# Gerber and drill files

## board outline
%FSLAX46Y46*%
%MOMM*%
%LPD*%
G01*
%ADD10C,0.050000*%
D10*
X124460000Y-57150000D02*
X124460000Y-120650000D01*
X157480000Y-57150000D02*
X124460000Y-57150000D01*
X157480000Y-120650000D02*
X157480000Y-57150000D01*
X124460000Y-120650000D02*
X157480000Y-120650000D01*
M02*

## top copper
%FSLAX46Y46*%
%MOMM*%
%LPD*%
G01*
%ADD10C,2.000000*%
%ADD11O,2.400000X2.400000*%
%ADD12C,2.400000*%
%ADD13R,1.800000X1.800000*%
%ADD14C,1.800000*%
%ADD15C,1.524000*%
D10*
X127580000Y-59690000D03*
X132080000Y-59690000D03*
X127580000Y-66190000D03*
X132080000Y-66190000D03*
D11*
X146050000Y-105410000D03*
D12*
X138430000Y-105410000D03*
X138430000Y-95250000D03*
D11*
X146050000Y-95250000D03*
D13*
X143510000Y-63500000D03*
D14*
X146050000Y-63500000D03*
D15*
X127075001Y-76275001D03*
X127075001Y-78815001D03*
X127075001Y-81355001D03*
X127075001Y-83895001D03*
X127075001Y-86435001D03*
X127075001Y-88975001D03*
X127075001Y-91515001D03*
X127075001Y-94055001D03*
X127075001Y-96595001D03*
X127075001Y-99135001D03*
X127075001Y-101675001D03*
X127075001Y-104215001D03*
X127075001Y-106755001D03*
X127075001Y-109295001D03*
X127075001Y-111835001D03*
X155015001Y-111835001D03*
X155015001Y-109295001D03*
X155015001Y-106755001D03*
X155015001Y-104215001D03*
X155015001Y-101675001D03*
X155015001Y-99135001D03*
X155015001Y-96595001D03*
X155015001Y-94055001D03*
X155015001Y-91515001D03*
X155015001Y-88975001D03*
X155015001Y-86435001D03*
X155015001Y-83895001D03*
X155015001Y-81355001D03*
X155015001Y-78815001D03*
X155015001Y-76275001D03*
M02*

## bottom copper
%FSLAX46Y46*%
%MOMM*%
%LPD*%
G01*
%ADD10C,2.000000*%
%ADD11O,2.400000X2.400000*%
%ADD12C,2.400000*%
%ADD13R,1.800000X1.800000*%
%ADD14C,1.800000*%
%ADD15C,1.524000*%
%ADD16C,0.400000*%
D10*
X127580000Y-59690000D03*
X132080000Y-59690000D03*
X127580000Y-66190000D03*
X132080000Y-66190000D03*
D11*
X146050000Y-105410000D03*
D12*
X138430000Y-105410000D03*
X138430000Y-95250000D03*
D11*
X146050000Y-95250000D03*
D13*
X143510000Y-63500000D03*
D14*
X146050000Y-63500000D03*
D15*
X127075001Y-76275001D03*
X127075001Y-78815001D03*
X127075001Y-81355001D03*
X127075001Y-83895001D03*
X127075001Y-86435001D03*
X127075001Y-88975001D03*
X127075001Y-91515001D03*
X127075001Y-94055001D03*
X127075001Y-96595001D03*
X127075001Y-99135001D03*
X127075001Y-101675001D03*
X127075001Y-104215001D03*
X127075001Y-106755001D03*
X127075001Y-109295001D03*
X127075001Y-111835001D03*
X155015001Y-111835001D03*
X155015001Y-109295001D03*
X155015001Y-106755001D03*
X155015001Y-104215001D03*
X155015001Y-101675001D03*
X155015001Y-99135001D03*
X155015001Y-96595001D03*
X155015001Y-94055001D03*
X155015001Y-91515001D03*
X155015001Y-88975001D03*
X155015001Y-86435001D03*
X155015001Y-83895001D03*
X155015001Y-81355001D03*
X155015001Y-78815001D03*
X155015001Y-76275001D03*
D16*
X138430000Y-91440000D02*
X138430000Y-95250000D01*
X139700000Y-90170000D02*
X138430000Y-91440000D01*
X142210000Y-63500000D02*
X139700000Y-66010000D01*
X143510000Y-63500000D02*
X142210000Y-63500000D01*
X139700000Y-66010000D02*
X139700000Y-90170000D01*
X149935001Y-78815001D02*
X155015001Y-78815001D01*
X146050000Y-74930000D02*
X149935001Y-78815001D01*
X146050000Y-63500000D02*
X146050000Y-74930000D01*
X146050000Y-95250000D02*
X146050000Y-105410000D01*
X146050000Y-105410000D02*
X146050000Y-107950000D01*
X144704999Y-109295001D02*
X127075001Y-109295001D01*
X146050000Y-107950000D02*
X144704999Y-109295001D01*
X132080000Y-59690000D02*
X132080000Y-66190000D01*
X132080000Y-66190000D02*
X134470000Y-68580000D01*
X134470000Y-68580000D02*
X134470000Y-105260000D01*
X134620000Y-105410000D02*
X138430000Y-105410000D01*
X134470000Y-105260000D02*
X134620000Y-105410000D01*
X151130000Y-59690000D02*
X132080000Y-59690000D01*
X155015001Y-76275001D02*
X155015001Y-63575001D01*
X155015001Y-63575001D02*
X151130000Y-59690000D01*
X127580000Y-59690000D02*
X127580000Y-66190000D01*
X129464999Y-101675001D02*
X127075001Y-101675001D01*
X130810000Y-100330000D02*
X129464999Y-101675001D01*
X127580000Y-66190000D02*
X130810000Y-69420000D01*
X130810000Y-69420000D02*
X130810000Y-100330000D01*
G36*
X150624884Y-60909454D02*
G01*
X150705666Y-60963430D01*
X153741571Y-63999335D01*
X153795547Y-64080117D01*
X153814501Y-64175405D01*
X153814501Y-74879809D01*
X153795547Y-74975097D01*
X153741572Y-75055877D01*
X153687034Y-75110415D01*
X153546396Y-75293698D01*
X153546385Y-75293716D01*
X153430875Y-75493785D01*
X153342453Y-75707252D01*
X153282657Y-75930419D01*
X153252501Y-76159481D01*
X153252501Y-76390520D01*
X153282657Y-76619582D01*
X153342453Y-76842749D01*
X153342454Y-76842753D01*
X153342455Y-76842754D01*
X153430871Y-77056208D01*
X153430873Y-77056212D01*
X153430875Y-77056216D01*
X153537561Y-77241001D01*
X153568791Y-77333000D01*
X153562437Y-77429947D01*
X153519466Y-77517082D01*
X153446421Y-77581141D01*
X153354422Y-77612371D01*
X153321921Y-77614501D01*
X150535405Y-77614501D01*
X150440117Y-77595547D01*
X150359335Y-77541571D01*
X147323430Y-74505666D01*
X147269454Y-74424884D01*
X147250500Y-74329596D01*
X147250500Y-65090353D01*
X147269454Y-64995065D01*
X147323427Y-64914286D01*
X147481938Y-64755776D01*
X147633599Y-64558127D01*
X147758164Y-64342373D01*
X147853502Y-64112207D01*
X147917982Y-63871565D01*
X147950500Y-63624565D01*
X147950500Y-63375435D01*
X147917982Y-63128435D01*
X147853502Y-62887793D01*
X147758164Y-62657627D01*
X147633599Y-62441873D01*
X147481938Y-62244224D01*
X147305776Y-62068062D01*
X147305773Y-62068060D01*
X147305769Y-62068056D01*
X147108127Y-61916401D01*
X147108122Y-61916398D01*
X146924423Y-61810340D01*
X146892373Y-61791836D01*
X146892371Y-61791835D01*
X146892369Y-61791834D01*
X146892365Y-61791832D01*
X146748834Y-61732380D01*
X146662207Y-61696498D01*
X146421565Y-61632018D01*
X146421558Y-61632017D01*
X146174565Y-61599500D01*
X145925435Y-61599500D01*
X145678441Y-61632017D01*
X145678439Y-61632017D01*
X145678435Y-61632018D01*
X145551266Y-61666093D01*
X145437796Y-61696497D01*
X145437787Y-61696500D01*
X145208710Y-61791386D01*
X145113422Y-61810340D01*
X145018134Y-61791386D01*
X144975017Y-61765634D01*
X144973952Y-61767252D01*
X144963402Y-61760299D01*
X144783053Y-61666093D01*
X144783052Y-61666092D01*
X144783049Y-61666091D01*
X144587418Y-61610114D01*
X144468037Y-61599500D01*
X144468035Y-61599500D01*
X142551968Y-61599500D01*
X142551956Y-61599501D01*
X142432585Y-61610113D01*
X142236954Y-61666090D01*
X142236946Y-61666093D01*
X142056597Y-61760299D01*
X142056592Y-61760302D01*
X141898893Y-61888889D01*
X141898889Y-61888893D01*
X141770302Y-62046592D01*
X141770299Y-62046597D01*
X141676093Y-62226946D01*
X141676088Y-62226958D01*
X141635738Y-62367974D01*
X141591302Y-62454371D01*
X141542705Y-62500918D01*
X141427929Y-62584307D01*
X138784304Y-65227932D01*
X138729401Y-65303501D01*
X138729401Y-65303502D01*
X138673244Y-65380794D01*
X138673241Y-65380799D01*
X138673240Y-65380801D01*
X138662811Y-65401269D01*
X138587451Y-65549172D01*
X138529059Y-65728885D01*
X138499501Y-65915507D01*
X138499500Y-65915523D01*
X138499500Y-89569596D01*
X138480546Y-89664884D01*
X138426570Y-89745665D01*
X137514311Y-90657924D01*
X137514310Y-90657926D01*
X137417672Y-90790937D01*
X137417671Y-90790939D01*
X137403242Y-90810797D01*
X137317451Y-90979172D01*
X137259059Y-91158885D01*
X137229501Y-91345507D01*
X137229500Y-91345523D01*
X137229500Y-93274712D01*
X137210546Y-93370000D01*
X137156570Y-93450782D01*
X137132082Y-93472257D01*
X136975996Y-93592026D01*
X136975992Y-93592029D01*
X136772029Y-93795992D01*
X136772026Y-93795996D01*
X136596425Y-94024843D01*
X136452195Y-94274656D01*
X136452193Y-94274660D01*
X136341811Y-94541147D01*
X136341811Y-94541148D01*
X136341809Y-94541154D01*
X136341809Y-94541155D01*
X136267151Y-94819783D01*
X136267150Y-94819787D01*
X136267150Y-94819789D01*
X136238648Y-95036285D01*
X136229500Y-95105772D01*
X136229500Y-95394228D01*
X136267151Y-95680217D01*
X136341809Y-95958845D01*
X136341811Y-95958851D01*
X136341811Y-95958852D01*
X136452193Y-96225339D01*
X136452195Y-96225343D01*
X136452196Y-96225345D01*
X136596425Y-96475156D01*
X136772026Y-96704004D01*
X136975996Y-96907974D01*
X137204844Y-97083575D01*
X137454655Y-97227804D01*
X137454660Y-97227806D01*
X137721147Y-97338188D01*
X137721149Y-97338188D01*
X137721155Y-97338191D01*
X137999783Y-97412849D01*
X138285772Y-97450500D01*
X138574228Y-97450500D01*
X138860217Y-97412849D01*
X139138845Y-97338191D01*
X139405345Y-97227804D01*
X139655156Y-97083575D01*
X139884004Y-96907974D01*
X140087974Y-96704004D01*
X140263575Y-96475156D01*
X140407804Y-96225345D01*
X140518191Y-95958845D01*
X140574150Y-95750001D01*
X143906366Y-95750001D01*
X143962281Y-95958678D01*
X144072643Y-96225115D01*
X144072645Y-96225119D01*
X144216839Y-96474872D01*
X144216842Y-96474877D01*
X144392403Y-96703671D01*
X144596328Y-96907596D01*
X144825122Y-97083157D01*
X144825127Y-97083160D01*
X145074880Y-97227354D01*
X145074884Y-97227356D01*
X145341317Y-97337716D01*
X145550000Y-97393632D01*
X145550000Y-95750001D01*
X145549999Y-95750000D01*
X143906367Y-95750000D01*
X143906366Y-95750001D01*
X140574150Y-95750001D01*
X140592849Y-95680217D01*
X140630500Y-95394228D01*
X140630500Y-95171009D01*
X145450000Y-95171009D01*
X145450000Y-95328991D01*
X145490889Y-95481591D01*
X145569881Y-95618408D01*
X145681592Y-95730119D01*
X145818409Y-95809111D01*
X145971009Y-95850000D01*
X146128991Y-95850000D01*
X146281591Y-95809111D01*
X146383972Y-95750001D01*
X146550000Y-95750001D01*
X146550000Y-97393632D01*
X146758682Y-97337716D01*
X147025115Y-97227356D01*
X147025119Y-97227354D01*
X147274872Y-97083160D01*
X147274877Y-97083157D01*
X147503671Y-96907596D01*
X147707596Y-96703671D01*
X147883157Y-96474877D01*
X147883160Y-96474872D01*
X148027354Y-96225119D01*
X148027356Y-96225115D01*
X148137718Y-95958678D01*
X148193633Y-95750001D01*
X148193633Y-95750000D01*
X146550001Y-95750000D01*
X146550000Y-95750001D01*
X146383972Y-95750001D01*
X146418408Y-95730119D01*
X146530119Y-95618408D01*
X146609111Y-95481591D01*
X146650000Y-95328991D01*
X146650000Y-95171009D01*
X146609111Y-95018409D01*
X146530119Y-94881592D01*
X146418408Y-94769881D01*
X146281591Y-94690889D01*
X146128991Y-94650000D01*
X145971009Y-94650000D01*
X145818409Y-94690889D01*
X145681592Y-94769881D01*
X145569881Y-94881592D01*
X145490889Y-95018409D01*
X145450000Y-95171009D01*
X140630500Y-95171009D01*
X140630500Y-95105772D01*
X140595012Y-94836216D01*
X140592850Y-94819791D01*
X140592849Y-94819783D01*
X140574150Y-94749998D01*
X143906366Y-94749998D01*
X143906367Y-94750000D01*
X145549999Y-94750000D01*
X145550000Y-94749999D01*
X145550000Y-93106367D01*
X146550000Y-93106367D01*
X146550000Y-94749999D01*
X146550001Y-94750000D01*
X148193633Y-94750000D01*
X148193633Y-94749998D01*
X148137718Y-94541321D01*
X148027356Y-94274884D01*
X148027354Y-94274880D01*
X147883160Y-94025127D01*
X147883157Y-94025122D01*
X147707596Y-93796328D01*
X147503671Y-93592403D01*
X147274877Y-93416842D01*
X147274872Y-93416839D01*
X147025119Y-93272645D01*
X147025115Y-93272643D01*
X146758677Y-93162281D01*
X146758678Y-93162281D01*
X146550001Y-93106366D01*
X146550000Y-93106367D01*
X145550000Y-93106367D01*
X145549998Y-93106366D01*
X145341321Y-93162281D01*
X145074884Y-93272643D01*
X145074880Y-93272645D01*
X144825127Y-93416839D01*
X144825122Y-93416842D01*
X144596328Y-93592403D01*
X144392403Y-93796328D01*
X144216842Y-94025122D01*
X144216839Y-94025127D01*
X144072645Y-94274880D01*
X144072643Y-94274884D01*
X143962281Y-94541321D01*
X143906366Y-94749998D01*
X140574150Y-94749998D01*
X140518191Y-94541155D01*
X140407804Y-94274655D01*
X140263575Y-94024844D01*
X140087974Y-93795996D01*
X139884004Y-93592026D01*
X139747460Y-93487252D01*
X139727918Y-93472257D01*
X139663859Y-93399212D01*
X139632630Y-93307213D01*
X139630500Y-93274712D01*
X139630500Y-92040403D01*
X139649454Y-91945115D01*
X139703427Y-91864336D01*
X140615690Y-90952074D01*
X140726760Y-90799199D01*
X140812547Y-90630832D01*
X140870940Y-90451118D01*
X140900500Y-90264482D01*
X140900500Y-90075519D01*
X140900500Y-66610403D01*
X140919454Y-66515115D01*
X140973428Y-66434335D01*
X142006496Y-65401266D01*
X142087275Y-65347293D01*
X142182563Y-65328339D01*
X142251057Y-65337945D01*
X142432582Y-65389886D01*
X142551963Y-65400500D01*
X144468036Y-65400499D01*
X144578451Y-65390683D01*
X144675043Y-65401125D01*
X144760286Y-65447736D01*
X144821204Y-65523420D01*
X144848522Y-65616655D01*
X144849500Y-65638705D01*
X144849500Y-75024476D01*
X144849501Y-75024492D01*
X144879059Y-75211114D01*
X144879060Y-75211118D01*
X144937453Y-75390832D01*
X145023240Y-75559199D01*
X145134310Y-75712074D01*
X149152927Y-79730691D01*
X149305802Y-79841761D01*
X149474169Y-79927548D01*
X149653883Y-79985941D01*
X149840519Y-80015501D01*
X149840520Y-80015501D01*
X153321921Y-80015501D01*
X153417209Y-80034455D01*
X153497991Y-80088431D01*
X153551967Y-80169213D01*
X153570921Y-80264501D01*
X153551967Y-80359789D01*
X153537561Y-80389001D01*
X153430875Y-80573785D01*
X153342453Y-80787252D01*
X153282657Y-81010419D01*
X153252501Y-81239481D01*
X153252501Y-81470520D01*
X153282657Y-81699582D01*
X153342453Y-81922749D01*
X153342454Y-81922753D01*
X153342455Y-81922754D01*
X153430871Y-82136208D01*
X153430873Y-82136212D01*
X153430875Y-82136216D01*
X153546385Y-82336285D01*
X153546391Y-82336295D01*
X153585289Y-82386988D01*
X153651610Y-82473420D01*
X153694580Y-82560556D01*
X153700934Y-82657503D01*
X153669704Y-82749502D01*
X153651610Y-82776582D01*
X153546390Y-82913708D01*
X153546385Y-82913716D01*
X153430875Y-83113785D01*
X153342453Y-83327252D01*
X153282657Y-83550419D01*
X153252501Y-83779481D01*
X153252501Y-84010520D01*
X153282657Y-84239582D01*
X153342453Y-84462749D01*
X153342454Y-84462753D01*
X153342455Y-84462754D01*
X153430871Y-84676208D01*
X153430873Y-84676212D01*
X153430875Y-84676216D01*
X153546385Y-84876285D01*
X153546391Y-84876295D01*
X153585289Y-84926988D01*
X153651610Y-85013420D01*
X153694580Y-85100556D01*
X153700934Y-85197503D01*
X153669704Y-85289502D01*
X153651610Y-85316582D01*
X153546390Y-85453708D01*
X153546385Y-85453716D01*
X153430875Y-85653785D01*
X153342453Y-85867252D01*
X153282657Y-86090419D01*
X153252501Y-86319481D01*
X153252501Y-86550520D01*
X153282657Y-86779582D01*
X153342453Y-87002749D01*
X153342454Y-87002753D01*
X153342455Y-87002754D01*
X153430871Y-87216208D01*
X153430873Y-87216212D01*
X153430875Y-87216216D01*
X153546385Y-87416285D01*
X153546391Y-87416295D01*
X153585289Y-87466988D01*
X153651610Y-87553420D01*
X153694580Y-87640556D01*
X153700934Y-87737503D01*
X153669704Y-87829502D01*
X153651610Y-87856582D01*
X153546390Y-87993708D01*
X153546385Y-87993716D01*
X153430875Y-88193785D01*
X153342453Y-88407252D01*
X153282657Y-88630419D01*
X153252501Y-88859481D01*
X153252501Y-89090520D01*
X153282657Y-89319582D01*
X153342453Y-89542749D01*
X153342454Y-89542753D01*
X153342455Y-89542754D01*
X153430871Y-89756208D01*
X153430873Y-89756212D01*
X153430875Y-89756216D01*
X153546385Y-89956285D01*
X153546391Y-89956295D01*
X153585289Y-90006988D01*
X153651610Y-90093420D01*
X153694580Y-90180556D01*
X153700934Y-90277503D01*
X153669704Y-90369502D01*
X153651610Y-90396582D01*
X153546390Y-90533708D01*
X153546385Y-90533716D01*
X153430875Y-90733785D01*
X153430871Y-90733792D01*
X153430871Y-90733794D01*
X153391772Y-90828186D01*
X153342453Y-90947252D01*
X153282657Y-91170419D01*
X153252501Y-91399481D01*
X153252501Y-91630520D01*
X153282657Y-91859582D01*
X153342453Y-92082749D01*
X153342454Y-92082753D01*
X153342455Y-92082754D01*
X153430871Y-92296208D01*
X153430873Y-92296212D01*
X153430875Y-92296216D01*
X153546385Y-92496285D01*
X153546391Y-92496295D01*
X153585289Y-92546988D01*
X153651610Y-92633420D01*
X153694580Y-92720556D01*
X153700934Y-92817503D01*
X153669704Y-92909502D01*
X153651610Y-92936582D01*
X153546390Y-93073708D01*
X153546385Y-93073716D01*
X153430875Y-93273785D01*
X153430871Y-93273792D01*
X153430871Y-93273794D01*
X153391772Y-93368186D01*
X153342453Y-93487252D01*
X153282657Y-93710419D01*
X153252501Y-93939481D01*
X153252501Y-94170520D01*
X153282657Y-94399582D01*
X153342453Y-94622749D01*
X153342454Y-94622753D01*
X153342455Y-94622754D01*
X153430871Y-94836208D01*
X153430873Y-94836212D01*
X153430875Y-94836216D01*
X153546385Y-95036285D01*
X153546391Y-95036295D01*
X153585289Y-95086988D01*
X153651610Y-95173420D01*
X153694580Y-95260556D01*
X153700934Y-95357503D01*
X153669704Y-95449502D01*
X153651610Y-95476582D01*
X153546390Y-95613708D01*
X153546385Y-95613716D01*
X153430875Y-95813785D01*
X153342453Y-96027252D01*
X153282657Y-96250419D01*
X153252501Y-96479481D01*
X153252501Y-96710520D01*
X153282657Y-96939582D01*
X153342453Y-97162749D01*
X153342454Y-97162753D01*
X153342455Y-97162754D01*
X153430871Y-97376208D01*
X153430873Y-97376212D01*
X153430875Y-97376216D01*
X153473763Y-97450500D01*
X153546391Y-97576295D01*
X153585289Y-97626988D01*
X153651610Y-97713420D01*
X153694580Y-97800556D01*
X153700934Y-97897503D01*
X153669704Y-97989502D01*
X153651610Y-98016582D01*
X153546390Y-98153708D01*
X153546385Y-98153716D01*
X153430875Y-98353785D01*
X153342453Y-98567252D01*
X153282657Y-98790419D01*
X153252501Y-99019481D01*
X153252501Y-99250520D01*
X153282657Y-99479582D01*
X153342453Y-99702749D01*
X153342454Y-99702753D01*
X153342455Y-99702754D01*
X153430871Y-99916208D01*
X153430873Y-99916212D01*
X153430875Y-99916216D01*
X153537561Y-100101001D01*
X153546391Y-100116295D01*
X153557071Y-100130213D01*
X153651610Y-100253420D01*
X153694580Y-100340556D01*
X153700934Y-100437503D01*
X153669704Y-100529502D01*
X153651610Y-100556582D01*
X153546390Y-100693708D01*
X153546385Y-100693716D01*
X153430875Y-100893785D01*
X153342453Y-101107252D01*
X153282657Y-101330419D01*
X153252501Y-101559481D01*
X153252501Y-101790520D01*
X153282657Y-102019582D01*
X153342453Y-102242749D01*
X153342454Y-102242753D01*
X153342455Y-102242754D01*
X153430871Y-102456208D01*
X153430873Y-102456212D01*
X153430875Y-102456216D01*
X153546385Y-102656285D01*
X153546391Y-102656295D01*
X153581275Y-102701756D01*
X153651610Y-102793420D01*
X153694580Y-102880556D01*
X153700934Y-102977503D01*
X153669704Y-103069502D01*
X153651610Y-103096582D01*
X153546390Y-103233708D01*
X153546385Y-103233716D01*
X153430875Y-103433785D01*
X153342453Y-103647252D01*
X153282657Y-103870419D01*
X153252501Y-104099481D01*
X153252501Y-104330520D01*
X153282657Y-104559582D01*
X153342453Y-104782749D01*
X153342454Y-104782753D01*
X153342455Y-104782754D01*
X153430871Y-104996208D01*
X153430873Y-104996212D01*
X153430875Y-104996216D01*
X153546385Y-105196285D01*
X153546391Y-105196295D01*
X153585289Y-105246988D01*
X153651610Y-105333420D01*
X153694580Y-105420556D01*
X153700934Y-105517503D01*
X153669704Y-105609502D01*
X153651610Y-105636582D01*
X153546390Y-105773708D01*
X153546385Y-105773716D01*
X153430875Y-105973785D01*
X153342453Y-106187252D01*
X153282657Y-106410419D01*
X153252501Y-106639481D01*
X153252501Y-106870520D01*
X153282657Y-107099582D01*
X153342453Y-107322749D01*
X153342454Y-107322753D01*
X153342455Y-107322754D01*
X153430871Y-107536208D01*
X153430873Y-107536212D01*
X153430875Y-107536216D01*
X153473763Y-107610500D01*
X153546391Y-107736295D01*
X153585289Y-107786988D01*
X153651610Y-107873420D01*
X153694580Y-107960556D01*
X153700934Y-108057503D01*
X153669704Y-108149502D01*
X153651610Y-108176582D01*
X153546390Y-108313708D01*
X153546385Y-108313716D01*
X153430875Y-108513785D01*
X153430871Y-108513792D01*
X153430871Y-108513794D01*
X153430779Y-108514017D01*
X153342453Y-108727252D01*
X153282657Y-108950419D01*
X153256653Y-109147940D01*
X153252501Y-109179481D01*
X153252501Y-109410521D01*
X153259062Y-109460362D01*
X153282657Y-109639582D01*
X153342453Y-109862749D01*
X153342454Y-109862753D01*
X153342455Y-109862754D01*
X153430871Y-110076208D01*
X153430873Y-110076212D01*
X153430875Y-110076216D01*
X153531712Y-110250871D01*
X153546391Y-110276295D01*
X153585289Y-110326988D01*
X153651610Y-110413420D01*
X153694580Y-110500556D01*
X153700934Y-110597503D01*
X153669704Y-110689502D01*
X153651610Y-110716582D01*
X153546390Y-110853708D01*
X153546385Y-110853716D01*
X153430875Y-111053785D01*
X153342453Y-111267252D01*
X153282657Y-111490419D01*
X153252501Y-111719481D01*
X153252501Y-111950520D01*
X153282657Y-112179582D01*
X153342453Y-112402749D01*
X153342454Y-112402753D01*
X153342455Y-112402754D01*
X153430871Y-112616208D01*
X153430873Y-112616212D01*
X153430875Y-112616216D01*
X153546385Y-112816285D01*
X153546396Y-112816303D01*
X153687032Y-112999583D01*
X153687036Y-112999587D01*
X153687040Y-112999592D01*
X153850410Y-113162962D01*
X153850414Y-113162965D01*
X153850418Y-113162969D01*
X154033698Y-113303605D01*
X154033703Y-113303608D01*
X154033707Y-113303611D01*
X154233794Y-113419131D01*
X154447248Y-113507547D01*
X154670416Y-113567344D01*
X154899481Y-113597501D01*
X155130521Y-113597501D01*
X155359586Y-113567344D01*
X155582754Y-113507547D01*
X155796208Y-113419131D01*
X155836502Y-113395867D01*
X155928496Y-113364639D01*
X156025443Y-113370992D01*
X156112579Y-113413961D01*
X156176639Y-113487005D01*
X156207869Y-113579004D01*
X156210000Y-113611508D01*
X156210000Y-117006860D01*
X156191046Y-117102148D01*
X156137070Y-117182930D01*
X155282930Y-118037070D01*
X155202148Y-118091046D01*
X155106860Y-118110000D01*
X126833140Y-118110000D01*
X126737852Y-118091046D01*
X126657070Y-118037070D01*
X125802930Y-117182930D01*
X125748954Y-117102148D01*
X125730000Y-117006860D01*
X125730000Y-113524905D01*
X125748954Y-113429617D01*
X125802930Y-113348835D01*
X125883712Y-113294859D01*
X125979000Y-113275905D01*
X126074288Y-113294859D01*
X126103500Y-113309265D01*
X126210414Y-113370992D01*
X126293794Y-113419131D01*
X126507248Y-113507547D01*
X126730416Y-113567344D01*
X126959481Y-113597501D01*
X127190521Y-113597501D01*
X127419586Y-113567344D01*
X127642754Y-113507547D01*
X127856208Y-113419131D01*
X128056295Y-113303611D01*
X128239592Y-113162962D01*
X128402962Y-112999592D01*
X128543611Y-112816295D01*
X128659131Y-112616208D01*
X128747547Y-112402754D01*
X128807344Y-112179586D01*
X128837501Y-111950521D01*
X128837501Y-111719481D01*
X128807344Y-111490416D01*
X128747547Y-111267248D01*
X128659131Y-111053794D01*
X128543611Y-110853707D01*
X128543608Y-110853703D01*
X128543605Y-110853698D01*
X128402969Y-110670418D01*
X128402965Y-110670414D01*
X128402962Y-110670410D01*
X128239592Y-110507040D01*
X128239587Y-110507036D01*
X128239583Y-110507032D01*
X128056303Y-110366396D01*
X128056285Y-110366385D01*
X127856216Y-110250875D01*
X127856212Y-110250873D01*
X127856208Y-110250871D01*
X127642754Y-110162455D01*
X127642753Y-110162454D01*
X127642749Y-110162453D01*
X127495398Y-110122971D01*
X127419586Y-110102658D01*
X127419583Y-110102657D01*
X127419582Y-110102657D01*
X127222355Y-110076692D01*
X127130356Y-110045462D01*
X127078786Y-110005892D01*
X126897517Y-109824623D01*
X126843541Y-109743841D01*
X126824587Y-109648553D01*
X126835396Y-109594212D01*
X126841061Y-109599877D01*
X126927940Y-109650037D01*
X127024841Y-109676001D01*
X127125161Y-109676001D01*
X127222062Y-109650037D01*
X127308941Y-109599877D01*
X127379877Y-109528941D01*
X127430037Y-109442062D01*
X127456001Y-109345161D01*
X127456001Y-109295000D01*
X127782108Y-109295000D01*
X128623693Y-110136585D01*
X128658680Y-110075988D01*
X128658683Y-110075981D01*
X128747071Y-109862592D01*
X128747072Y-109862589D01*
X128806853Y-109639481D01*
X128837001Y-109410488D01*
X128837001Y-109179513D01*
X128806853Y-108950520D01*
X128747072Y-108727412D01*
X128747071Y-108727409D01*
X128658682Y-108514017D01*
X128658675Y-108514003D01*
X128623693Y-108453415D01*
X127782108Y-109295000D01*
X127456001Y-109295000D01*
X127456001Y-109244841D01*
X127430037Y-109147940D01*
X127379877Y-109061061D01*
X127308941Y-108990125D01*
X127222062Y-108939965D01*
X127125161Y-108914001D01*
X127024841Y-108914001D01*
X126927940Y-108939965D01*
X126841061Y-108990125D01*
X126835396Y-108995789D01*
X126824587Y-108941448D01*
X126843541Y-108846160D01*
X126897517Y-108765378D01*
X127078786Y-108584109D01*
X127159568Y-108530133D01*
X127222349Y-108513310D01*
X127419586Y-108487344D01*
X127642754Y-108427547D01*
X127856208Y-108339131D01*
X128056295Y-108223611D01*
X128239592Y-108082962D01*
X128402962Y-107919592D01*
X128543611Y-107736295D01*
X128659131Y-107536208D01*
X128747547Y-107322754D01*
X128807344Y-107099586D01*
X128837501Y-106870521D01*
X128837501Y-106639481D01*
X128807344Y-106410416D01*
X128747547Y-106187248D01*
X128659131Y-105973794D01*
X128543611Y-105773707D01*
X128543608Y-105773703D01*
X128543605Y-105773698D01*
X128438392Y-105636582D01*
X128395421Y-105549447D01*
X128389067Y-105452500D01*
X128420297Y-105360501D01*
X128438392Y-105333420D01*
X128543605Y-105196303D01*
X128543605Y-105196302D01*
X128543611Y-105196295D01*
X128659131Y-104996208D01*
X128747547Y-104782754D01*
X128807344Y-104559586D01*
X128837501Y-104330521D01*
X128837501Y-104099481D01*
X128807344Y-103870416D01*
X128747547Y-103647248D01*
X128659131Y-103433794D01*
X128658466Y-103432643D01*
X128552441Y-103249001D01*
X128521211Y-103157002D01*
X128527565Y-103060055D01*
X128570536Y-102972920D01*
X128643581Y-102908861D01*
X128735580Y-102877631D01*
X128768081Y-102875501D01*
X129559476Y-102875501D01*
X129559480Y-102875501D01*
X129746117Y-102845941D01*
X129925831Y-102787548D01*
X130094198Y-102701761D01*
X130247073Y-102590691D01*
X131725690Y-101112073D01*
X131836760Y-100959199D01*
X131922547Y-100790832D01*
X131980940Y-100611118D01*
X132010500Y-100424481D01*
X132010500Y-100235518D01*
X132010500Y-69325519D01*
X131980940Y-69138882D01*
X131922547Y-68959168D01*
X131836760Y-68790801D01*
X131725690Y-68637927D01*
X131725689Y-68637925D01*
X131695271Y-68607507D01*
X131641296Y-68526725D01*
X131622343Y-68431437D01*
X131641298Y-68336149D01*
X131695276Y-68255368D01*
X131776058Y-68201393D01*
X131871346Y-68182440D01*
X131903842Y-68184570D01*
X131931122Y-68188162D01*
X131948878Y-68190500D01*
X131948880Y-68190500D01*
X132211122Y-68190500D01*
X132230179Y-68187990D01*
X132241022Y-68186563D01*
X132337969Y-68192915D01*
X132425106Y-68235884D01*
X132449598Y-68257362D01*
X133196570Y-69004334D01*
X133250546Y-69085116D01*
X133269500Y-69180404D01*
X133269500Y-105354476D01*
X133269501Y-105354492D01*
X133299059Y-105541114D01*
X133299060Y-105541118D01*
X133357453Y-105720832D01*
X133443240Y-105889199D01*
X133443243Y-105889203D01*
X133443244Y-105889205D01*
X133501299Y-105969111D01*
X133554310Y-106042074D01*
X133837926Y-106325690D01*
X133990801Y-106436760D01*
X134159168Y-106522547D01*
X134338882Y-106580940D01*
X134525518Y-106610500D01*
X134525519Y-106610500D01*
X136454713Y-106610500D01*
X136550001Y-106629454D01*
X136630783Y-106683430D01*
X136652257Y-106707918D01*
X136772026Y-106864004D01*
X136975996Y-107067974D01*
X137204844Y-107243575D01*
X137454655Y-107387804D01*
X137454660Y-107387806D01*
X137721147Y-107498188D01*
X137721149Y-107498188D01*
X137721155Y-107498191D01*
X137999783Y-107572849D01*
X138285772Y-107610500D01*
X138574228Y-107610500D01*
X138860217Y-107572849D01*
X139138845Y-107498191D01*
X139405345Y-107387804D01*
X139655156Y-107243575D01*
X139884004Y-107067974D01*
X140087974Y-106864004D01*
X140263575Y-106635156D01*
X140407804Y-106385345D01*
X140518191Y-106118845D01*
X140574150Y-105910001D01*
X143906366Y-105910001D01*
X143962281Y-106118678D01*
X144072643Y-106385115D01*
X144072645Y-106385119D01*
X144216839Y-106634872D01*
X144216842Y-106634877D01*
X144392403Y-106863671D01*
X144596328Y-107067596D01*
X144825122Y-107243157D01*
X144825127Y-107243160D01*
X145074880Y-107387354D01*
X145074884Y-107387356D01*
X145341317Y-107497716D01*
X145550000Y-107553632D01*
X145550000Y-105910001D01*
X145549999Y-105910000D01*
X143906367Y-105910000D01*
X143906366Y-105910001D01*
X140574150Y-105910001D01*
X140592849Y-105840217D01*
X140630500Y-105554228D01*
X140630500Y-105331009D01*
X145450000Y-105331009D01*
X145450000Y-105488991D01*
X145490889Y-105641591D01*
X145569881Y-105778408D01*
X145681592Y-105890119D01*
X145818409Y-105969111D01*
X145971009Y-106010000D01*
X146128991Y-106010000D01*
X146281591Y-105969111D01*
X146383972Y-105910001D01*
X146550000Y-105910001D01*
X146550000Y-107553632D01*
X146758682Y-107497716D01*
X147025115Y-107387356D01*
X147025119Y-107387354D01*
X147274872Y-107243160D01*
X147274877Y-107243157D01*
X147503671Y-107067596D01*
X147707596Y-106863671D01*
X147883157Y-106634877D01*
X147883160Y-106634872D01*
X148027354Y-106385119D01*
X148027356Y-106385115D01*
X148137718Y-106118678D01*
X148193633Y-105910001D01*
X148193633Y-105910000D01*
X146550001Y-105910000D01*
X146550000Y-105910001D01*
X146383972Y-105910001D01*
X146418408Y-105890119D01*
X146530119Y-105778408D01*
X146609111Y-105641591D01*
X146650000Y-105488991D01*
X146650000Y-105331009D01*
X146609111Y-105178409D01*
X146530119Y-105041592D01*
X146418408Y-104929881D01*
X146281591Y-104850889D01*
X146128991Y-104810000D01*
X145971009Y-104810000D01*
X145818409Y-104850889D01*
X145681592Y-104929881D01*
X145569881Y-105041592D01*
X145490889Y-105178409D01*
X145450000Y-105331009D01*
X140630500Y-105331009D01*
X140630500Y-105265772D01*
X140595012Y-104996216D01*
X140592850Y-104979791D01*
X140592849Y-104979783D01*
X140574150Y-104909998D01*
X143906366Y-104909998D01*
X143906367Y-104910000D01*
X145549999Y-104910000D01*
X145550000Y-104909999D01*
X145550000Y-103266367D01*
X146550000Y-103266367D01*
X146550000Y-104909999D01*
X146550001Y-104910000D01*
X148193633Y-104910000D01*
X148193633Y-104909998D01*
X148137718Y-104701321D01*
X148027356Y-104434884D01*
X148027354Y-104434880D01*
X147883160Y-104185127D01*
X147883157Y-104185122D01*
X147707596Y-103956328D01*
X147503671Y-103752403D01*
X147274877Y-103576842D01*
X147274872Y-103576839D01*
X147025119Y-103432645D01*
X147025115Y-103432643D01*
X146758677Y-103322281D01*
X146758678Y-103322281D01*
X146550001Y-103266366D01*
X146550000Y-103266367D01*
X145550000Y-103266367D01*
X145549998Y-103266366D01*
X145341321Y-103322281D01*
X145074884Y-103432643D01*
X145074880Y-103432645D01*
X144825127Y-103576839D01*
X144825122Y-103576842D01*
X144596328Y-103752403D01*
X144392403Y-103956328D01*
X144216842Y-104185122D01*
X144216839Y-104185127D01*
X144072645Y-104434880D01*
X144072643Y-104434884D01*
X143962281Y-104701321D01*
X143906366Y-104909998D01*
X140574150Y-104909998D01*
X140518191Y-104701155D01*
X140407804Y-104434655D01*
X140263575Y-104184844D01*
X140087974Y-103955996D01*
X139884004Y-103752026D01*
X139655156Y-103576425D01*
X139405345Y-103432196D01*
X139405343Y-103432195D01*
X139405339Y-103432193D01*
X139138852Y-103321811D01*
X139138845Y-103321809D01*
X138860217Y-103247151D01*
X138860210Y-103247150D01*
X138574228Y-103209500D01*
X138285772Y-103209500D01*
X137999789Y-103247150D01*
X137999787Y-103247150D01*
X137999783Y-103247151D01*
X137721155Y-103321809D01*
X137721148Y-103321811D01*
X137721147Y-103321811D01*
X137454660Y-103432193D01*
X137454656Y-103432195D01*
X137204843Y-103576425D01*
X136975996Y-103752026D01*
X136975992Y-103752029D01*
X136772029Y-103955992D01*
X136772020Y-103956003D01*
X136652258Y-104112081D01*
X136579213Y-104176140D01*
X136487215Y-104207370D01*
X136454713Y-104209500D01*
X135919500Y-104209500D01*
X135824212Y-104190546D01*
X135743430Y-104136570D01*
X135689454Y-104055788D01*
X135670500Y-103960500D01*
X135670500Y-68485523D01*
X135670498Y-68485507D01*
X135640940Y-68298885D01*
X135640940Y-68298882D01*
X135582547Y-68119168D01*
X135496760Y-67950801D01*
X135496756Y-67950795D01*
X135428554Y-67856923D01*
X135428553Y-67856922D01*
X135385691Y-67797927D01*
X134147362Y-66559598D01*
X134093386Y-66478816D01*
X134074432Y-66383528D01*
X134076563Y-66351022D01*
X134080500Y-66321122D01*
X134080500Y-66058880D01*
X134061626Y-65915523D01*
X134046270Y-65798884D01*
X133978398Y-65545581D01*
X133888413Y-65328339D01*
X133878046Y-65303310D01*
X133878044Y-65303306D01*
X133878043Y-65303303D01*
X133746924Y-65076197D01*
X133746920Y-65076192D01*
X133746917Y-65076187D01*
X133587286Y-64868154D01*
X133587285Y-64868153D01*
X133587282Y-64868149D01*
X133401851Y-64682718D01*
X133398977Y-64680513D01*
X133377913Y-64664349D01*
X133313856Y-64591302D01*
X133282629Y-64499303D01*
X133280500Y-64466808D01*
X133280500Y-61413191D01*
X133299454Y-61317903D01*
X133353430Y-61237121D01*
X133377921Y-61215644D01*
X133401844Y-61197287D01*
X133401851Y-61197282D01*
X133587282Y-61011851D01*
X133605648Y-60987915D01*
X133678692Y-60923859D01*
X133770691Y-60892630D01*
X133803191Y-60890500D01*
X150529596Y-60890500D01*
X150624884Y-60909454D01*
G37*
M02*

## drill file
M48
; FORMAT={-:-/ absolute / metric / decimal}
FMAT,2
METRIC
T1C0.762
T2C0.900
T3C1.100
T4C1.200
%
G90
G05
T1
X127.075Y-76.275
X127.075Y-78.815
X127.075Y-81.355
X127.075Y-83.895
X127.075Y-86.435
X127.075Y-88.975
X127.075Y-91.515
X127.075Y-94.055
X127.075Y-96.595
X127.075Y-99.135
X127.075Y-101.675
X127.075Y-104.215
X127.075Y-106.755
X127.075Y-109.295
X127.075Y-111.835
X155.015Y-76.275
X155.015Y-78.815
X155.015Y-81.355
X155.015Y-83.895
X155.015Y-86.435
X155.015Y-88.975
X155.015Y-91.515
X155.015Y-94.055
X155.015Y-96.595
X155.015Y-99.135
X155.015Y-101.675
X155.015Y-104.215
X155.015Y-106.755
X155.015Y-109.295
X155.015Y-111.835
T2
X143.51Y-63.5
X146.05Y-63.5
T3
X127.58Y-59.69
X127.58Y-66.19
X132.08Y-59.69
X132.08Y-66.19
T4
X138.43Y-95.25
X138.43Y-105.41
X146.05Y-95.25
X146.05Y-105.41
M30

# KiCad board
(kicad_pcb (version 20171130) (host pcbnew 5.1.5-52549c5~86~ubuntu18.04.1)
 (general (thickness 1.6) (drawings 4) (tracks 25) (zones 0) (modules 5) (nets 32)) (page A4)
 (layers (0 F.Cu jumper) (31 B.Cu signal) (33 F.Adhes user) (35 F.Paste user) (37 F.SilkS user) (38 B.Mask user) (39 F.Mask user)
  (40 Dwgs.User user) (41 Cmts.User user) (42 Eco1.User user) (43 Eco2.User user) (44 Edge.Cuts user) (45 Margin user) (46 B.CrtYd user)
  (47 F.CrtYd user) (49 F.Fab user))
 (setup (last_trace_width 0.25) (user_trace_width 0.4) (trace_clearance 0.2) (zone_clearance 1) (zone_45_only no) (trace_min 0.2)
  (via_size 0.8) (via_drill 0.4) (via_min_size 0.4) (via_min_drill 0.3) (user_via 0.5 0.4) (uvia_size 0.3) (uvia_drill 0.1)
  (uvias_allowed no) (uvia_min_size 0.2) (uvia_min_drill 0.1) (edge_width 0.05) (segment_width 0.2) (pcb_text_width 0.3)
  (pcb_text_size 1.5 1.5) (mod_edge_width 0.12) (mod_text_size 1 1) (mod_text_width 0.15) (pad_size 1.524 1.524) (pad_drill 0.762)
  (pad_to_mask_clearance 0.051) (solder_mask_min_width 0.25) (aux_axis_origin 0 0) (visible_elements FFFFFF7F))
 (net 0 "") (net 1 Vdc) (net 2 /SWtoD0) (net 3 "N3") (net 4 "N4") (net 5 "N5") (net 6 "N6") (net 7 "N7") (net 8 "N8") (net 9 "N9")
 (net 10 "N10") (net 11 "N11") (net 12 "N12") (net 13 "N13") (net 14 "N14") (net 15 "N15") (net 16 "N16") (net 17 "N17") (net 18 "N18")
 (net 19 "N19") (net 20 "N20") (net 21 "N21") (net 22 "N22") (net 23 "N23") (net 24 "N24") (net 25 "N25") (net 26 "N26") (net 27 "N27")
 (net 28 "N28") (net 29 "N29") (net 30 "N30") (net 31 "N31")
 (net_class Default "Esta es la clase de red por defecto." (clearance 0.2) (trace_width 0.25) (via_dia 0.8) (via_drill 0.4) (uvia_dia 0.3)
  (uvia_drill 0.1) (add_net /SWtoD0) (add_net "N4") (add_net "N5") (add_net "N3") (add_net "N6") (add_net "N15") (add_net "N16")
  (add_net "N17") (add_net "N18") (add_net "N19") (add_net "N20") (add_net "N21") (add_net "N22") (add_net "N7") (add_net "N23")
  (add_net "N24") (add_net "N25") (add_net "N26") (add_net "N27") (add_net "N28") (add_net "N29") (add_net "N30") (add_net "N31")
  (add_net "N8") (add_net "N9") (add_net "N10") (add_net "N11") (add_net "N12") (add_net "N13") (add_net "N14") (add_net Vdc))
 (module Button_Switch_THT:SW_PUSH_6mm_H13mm (layer F.Cu) (at 132.08 59.69 270)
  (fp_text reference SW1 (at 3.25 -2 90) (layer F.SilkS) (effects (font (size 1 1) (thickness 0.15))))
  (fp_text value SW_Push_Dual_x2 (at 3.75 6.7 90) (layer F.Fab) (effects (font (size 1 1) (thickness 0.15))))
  (pad 2 thru_hole circle (at 0 4.5) (size 2 2) (drill 1.1) (layers *.Cu *.Mask) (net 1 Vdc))
  (pad 1 thru_hole circle (at 0 0) (size 2 2) (drill 1.1) (layers *.Cu *.Mask) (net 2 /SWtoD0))
  (pad 2 thru_hole circle (at 6.5 4.5) (size 2 2) (drill 1.1) (layers *.Cu *.Mask) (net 1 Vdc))
  (pad 1 thru_hole circle (at 6.5 0) (size 2 2) (drill 1.1) (layers *.Cu *.Mask) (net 2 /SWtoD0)))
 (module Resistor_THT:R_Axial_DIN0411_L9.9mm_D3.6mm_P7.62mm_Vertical (layer F.Cu) (at 138.43 105.41)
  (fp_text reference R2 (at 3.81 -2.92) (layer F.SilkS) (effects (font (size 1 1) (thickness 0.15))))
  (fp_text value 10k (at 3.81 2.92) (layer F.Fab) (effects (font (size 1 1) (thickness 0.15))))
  (pad 2 thru_hole oval (at 7.62 0) (size 2.4 2.4) (drill 1.2) (layers *.Cu *.Mask) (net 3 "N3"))
  (pad 1 thru_hole circle (at 0 0) (size 2.4 2.4) (drill 1.2) (layers *.Cu *.Mask) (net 2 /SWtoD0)))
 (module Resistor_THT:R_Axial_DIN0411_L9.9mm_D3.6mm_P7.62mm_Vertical (layer F.Cu) (at 138.43 95.25)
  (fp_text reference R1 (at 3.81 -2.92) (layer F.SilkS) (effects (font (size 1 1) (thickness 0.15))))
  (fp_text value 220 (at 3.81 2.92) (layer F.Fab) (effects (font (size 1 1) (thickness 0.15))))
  (pad 1 thru_hole circle (at 0 0) (size 2.4 2.4) (drill 1.2) (layers *.Cu *.Mask) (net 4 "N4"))
  (pad 2 thru_hole oval (at 7.62 0) (size 2.4 2.4) (drill 1.2) (layers *.Cu *.Mask) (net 3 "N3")))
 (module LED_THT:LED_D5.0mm (layer F.Cu) (at 143.51 63.5)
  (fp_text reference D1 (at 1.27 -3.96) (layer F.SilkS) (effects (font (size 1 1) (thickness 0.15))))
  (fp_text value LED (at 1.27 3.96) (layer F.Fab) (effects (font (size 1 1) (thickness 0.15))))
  (pad 1 thru_hole rect (at 0 0) (size 1.8 1.8) (drill 0.9) (layers *.Cu *.Mask) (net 4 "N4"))
  (pad 2 thru_hole circle (at 2.54 0) (size 1.8 1.8) (drill 0.9) (layers *.Cu *.Mask) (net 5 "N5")))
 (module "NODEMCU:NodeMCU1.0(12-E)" (layer F.Cu) (at 141.045001 94.055001)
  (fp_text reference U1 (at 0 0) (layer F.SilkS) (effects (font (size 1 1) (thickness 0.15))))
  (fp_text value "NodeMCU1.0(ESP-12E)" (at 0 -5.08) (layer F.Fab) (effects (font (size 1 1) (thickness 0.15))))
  (pad 1 thru_hole circle (at -13.97 -17.78) (size 1.524 1.524) (drill 0.762) (layers *.Cu *.Mask F.SilkS) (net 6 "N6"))
  (pad 2 thru_hole circle (at -13.97 -15.24) (size 1.524 1.524) (drill 0.762) (layers *.Cu *.Mask F.SilkS) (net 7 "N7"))
  (pad 3 thru_hole circle (at -13.97 -12.7) (size 1.524 1.524) (drill 0.762) (layers *.Cu *.Mask F.SilkS) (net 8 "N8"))
  (pad 4 thru_hole circle (at -13.97 -10.16) (size 1.524 1.524) (drill 0.762) (layers *.Cu *.Mask F.SilkS) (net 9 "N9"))
  (pad 5 thru_hole circle (at -13.97 -7.62) (size 1.524 1.524) (drill 0.762) (layers *.Cu *.Mask F.SilkS) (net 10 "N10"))
  (pad 6 thru_hole circle (at -13.97 -5.08) (size 1.524 1.524) (drill 0.762) (layers *.Cu *.Mask F.SilkS) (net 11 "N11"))
  (pad 7 thru_hole circle (at -13.97 -2.54) (size 1.524 1.524) (drill 0.762) (layers *.Cu *.Mask F.SilkS) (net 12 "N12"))
  (pad 8 thru_hole circle (at -13.97 0) (size 1.524 1.524) (drill 0.762) (layers *.Cu *.Mask F.SilkS) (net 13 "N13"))
  (pad 9 thru_hole circle (at -13.97 2.54) (size 1.524 1.524) (drill 0.762) (layers *.Cu *.Mask F.SilkS) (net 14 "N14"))
  (pad 10 thru_hole circle (at -13.97 5.08) (size 1.524 1.524) (drill 0.762) (layers *.Cu *.Mask F.SilkS) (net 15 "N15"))
  (pad 11 thru_hole circle (at -13.97 7.62) (size 1.524 1.524) (drill 0.762) (layers *.Cu *.Mask F.SilkS) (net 1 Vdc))
  (pad 12 thru_hole circle (at -13.97 10.16) (size 1.524 1.524) (drill 0.762) (layers *.Cu *.Mask F.SilkS) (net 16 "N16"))
  (pad 13 thru_hole circle (at -13.97 12.7) (size 1.524 1.524) (drill 0.762) (layers *.Cu *.Mask F.SilkS) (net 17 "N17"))
  (pad 14 thru_hole circle (at -13.97 15.24) (size 1.524 1.524) (drill 0.762) (layers *.Cu *.Mask F.SilkS) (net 3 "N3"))
  (pad 15 thru_hole circle (at -13.97 17.78) (size 1.524 1.524) (drill 0.762) (layers *.Cu *.Mask F.SilkS) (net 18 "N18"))
  (pad 16 thru_hole circle (at 13.97 17.78) (size 1.524 1.524) (drill 0.762) (layers *.Cu *.Mask F.SilkS) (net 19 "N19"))
  (pad 17 thru_hole circle (at 13.97 15.24) (size 1.524 1.524) (drill 0.762) (layers *.Cu *.Mask F.SilkS) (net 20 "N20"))
  (pad 18 thru_hole circle (at 13.97 12.7) (size 1.524 1.524) (drill 0.762) (layers *.Cu *.Mask F.SilkS) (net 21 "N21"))
  (pad 19 thru_hole circle (at 13.97 10.16) (size 1.524 1.524) (drill 0.762) (layers *.Cu *.Mask F.SilkS) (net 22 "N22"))
  (pad 20 thru_hole circle (at 13.97 7.62) (size 1.524 1.524) (drill 0.762) (layers *.Cu *.Mask F.SilkS) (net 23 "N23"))
  (pad 21 thru_hole circle (at 13.97 5.08) (size 1.524 1.524) (drill 0.762) (layers *.Cu *.Mask F.SilkS) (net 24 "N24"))
  (pad 22 thru_hole circle (at 13.97 2.54) (size 1.524 1.524) (drill 0.762) (layers *.Cu *.Mask F.SilkS) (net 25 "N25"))
  (pad 23 thru_hole circle (at 13.97 0) (size 1.524 1.524) (drill 0.762) (layers *.Cu *.Mask F.SilkS) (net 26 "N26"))
  (pad 24 thru_hole circle (at 13.97 -2.54) (size 1.524 1.524) (drill 0.762) (layers *.Cu *.Mask F.SilkS) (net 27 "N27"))
  (pad 25 thru_hole circle (at 13.97 -5.08) (size 1.524 1.524) (drill 0.762) (layers *.Cu *.Mask F.SilkS) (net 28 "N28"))
  (pad 26 thru_hole circle (at 13.97 -7.62) (size 1.524 1.524) (drill 0.762) (layers *.Cu *.Mask F.SilkS) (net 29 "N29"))
  (pad 27 thru_hole circle (at 13.97 -10.16) (size 1.524 1.524) (drill 0.762) (layers *.Cu *.Mask F.SilkS) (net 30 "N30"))
  (pad 28 thru_hole circle (at 13.97 -12.7) (size 1.524 1.524) (drill 0.762) (layers *.Cu *.Mask F.SilkS) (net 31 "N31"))
  (pad 29 thru_hole circle (at 13.97 -15.24) (size 1.524 1.524) (drill 0.762) (layers *.Cu *.Mask F.SilkS) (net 5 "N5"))
  (pad 30 thru_hole circle (at 13.97 -17.78) (size 1.524 1.524) (drill 0.762) (layers *.Cu *.Mask F.SilkS) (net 2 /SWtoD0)))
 (gr_line (start 124.46 57.15) (end 124.46 120.65) (layer Edge.Cuts) (width 0.05))
 (gr_line (start 157.48 57.15) (end 124.46 57.15) (layer Edge.Cuts) (width 0.05))
 (gr_line (start 157.48 120.65) (end 157.48 57.15) (layer Edge.Cuts) (width 0.05))
 (gr_line (start 124.46 120.65) (end 157.48 120.65) (layer Edge.Cuts) (width 0.05))
 (segment (start 138.43 91.44) (end 138.43 95.25) (width 0.4) (layer B.Cu) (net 4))
 (segment (start 139.7 90.17) (end 138.43 91.44) (width 0.4) (layer B.Cu) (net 4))
 (segment (start 142.21 63.5) (end 139.7 66.01) (width 0.4) (layer B.Cu) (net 4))
 (segment (start 143.51 63.5) (end 142.21 63.5) (width 0.4) (layer B.Cu) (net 4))
 (segment (start 139.7 66.01) (end 139.7 90.17) (width 0.4) (layer B.Cu) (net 4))
 (segment (start 149.935001 78.815001) (end 155.015001 78.815001) (width 0.4) (layer B.Cu) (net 5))
 (segment (start 146.05 74.93) (end 149.935001 78.815001) (width 0.4) (layer B.Cu) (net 5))
 (segment (start 146.05 63.5) (end 146.05 74.93) (width 0.4) (layer B.Cu) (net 5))
 (segment (start 146.05 95.25) (end 146.05 105.41) (width 0.4) (layer B.Cu) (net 3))
 (segment (start 146.05 105.41) (end 146.05 107.95) (width 0.4) (layer B.Cu) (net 3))
 (segment (start 144.704999 109.295001) (end 127.075001 109.295001) (width 0.4) (layer B.Cu) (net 3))
 (segment (start 146.05 107.95) (end 144.704999 109.295001) (width 0.4) (layer B.Cu) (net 3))
 (segment (start 132.08 59.69) (end 132.08 66.19) (width 0.4) (layer B.Cu) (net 2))
 (segment (start 132.08 66.19) (end 134.47 68.58) (width 0.4) (layer B.Cu) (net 2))
 (segment (start 134.47 68.58) (end 134.47 105.26) (width 0.4) (layer B.Cu) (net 2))
 (segment (start 134.62 105.41) (end 138.43 105.41) (width 0.4) (layer B.Cu) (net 2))
 (segment (start 134.47 105.26) (end 134.62 105.41) (width 0.4) (layer B.Cu) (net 2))
 (segment (start 151.13 59.69) (end 132.08 59.69) (width 0.4) (layer B.Cu) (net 2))
 (segment (start 155.015001 76.275001) (end 155.015001 63.575001) (width 0.4) (layer B.Cu) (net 2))
 (segment (start 155.015001 63.575001) (end 151.13 59.69) (width 0.4) (layer B.Cu) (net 2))
 (segment (start 127.58 59.69) (end 127.58 66.19) (width 0.4) (layer B.Cu) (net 1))
 (segment (start 129.464999 101.675001) (end 127.075001 101.675001) (width 0.4) (layer B.Cu) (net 1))
 (segment (start 130.81 100.33) (end 129.464999 101.675001) (width 0.4) (layer B.Cu) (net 1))
 (segment (start 127.58 66.19) (end 130.81 69.42) (width 0.4) (layer B.Cu) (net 1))
 (segment (start 130.81 69.42) (end 130.81 100.33) (width 0.4) (layer B.Cu) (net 1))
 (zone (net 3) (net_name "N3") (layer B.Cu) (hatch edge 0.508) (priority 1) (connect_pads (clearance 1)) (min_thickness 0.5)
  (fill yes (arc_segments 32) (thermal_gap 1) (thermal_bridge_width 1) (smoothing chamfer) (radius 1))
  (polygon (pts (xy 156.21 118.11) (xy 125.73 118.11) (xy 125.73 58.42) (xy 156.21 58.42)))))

